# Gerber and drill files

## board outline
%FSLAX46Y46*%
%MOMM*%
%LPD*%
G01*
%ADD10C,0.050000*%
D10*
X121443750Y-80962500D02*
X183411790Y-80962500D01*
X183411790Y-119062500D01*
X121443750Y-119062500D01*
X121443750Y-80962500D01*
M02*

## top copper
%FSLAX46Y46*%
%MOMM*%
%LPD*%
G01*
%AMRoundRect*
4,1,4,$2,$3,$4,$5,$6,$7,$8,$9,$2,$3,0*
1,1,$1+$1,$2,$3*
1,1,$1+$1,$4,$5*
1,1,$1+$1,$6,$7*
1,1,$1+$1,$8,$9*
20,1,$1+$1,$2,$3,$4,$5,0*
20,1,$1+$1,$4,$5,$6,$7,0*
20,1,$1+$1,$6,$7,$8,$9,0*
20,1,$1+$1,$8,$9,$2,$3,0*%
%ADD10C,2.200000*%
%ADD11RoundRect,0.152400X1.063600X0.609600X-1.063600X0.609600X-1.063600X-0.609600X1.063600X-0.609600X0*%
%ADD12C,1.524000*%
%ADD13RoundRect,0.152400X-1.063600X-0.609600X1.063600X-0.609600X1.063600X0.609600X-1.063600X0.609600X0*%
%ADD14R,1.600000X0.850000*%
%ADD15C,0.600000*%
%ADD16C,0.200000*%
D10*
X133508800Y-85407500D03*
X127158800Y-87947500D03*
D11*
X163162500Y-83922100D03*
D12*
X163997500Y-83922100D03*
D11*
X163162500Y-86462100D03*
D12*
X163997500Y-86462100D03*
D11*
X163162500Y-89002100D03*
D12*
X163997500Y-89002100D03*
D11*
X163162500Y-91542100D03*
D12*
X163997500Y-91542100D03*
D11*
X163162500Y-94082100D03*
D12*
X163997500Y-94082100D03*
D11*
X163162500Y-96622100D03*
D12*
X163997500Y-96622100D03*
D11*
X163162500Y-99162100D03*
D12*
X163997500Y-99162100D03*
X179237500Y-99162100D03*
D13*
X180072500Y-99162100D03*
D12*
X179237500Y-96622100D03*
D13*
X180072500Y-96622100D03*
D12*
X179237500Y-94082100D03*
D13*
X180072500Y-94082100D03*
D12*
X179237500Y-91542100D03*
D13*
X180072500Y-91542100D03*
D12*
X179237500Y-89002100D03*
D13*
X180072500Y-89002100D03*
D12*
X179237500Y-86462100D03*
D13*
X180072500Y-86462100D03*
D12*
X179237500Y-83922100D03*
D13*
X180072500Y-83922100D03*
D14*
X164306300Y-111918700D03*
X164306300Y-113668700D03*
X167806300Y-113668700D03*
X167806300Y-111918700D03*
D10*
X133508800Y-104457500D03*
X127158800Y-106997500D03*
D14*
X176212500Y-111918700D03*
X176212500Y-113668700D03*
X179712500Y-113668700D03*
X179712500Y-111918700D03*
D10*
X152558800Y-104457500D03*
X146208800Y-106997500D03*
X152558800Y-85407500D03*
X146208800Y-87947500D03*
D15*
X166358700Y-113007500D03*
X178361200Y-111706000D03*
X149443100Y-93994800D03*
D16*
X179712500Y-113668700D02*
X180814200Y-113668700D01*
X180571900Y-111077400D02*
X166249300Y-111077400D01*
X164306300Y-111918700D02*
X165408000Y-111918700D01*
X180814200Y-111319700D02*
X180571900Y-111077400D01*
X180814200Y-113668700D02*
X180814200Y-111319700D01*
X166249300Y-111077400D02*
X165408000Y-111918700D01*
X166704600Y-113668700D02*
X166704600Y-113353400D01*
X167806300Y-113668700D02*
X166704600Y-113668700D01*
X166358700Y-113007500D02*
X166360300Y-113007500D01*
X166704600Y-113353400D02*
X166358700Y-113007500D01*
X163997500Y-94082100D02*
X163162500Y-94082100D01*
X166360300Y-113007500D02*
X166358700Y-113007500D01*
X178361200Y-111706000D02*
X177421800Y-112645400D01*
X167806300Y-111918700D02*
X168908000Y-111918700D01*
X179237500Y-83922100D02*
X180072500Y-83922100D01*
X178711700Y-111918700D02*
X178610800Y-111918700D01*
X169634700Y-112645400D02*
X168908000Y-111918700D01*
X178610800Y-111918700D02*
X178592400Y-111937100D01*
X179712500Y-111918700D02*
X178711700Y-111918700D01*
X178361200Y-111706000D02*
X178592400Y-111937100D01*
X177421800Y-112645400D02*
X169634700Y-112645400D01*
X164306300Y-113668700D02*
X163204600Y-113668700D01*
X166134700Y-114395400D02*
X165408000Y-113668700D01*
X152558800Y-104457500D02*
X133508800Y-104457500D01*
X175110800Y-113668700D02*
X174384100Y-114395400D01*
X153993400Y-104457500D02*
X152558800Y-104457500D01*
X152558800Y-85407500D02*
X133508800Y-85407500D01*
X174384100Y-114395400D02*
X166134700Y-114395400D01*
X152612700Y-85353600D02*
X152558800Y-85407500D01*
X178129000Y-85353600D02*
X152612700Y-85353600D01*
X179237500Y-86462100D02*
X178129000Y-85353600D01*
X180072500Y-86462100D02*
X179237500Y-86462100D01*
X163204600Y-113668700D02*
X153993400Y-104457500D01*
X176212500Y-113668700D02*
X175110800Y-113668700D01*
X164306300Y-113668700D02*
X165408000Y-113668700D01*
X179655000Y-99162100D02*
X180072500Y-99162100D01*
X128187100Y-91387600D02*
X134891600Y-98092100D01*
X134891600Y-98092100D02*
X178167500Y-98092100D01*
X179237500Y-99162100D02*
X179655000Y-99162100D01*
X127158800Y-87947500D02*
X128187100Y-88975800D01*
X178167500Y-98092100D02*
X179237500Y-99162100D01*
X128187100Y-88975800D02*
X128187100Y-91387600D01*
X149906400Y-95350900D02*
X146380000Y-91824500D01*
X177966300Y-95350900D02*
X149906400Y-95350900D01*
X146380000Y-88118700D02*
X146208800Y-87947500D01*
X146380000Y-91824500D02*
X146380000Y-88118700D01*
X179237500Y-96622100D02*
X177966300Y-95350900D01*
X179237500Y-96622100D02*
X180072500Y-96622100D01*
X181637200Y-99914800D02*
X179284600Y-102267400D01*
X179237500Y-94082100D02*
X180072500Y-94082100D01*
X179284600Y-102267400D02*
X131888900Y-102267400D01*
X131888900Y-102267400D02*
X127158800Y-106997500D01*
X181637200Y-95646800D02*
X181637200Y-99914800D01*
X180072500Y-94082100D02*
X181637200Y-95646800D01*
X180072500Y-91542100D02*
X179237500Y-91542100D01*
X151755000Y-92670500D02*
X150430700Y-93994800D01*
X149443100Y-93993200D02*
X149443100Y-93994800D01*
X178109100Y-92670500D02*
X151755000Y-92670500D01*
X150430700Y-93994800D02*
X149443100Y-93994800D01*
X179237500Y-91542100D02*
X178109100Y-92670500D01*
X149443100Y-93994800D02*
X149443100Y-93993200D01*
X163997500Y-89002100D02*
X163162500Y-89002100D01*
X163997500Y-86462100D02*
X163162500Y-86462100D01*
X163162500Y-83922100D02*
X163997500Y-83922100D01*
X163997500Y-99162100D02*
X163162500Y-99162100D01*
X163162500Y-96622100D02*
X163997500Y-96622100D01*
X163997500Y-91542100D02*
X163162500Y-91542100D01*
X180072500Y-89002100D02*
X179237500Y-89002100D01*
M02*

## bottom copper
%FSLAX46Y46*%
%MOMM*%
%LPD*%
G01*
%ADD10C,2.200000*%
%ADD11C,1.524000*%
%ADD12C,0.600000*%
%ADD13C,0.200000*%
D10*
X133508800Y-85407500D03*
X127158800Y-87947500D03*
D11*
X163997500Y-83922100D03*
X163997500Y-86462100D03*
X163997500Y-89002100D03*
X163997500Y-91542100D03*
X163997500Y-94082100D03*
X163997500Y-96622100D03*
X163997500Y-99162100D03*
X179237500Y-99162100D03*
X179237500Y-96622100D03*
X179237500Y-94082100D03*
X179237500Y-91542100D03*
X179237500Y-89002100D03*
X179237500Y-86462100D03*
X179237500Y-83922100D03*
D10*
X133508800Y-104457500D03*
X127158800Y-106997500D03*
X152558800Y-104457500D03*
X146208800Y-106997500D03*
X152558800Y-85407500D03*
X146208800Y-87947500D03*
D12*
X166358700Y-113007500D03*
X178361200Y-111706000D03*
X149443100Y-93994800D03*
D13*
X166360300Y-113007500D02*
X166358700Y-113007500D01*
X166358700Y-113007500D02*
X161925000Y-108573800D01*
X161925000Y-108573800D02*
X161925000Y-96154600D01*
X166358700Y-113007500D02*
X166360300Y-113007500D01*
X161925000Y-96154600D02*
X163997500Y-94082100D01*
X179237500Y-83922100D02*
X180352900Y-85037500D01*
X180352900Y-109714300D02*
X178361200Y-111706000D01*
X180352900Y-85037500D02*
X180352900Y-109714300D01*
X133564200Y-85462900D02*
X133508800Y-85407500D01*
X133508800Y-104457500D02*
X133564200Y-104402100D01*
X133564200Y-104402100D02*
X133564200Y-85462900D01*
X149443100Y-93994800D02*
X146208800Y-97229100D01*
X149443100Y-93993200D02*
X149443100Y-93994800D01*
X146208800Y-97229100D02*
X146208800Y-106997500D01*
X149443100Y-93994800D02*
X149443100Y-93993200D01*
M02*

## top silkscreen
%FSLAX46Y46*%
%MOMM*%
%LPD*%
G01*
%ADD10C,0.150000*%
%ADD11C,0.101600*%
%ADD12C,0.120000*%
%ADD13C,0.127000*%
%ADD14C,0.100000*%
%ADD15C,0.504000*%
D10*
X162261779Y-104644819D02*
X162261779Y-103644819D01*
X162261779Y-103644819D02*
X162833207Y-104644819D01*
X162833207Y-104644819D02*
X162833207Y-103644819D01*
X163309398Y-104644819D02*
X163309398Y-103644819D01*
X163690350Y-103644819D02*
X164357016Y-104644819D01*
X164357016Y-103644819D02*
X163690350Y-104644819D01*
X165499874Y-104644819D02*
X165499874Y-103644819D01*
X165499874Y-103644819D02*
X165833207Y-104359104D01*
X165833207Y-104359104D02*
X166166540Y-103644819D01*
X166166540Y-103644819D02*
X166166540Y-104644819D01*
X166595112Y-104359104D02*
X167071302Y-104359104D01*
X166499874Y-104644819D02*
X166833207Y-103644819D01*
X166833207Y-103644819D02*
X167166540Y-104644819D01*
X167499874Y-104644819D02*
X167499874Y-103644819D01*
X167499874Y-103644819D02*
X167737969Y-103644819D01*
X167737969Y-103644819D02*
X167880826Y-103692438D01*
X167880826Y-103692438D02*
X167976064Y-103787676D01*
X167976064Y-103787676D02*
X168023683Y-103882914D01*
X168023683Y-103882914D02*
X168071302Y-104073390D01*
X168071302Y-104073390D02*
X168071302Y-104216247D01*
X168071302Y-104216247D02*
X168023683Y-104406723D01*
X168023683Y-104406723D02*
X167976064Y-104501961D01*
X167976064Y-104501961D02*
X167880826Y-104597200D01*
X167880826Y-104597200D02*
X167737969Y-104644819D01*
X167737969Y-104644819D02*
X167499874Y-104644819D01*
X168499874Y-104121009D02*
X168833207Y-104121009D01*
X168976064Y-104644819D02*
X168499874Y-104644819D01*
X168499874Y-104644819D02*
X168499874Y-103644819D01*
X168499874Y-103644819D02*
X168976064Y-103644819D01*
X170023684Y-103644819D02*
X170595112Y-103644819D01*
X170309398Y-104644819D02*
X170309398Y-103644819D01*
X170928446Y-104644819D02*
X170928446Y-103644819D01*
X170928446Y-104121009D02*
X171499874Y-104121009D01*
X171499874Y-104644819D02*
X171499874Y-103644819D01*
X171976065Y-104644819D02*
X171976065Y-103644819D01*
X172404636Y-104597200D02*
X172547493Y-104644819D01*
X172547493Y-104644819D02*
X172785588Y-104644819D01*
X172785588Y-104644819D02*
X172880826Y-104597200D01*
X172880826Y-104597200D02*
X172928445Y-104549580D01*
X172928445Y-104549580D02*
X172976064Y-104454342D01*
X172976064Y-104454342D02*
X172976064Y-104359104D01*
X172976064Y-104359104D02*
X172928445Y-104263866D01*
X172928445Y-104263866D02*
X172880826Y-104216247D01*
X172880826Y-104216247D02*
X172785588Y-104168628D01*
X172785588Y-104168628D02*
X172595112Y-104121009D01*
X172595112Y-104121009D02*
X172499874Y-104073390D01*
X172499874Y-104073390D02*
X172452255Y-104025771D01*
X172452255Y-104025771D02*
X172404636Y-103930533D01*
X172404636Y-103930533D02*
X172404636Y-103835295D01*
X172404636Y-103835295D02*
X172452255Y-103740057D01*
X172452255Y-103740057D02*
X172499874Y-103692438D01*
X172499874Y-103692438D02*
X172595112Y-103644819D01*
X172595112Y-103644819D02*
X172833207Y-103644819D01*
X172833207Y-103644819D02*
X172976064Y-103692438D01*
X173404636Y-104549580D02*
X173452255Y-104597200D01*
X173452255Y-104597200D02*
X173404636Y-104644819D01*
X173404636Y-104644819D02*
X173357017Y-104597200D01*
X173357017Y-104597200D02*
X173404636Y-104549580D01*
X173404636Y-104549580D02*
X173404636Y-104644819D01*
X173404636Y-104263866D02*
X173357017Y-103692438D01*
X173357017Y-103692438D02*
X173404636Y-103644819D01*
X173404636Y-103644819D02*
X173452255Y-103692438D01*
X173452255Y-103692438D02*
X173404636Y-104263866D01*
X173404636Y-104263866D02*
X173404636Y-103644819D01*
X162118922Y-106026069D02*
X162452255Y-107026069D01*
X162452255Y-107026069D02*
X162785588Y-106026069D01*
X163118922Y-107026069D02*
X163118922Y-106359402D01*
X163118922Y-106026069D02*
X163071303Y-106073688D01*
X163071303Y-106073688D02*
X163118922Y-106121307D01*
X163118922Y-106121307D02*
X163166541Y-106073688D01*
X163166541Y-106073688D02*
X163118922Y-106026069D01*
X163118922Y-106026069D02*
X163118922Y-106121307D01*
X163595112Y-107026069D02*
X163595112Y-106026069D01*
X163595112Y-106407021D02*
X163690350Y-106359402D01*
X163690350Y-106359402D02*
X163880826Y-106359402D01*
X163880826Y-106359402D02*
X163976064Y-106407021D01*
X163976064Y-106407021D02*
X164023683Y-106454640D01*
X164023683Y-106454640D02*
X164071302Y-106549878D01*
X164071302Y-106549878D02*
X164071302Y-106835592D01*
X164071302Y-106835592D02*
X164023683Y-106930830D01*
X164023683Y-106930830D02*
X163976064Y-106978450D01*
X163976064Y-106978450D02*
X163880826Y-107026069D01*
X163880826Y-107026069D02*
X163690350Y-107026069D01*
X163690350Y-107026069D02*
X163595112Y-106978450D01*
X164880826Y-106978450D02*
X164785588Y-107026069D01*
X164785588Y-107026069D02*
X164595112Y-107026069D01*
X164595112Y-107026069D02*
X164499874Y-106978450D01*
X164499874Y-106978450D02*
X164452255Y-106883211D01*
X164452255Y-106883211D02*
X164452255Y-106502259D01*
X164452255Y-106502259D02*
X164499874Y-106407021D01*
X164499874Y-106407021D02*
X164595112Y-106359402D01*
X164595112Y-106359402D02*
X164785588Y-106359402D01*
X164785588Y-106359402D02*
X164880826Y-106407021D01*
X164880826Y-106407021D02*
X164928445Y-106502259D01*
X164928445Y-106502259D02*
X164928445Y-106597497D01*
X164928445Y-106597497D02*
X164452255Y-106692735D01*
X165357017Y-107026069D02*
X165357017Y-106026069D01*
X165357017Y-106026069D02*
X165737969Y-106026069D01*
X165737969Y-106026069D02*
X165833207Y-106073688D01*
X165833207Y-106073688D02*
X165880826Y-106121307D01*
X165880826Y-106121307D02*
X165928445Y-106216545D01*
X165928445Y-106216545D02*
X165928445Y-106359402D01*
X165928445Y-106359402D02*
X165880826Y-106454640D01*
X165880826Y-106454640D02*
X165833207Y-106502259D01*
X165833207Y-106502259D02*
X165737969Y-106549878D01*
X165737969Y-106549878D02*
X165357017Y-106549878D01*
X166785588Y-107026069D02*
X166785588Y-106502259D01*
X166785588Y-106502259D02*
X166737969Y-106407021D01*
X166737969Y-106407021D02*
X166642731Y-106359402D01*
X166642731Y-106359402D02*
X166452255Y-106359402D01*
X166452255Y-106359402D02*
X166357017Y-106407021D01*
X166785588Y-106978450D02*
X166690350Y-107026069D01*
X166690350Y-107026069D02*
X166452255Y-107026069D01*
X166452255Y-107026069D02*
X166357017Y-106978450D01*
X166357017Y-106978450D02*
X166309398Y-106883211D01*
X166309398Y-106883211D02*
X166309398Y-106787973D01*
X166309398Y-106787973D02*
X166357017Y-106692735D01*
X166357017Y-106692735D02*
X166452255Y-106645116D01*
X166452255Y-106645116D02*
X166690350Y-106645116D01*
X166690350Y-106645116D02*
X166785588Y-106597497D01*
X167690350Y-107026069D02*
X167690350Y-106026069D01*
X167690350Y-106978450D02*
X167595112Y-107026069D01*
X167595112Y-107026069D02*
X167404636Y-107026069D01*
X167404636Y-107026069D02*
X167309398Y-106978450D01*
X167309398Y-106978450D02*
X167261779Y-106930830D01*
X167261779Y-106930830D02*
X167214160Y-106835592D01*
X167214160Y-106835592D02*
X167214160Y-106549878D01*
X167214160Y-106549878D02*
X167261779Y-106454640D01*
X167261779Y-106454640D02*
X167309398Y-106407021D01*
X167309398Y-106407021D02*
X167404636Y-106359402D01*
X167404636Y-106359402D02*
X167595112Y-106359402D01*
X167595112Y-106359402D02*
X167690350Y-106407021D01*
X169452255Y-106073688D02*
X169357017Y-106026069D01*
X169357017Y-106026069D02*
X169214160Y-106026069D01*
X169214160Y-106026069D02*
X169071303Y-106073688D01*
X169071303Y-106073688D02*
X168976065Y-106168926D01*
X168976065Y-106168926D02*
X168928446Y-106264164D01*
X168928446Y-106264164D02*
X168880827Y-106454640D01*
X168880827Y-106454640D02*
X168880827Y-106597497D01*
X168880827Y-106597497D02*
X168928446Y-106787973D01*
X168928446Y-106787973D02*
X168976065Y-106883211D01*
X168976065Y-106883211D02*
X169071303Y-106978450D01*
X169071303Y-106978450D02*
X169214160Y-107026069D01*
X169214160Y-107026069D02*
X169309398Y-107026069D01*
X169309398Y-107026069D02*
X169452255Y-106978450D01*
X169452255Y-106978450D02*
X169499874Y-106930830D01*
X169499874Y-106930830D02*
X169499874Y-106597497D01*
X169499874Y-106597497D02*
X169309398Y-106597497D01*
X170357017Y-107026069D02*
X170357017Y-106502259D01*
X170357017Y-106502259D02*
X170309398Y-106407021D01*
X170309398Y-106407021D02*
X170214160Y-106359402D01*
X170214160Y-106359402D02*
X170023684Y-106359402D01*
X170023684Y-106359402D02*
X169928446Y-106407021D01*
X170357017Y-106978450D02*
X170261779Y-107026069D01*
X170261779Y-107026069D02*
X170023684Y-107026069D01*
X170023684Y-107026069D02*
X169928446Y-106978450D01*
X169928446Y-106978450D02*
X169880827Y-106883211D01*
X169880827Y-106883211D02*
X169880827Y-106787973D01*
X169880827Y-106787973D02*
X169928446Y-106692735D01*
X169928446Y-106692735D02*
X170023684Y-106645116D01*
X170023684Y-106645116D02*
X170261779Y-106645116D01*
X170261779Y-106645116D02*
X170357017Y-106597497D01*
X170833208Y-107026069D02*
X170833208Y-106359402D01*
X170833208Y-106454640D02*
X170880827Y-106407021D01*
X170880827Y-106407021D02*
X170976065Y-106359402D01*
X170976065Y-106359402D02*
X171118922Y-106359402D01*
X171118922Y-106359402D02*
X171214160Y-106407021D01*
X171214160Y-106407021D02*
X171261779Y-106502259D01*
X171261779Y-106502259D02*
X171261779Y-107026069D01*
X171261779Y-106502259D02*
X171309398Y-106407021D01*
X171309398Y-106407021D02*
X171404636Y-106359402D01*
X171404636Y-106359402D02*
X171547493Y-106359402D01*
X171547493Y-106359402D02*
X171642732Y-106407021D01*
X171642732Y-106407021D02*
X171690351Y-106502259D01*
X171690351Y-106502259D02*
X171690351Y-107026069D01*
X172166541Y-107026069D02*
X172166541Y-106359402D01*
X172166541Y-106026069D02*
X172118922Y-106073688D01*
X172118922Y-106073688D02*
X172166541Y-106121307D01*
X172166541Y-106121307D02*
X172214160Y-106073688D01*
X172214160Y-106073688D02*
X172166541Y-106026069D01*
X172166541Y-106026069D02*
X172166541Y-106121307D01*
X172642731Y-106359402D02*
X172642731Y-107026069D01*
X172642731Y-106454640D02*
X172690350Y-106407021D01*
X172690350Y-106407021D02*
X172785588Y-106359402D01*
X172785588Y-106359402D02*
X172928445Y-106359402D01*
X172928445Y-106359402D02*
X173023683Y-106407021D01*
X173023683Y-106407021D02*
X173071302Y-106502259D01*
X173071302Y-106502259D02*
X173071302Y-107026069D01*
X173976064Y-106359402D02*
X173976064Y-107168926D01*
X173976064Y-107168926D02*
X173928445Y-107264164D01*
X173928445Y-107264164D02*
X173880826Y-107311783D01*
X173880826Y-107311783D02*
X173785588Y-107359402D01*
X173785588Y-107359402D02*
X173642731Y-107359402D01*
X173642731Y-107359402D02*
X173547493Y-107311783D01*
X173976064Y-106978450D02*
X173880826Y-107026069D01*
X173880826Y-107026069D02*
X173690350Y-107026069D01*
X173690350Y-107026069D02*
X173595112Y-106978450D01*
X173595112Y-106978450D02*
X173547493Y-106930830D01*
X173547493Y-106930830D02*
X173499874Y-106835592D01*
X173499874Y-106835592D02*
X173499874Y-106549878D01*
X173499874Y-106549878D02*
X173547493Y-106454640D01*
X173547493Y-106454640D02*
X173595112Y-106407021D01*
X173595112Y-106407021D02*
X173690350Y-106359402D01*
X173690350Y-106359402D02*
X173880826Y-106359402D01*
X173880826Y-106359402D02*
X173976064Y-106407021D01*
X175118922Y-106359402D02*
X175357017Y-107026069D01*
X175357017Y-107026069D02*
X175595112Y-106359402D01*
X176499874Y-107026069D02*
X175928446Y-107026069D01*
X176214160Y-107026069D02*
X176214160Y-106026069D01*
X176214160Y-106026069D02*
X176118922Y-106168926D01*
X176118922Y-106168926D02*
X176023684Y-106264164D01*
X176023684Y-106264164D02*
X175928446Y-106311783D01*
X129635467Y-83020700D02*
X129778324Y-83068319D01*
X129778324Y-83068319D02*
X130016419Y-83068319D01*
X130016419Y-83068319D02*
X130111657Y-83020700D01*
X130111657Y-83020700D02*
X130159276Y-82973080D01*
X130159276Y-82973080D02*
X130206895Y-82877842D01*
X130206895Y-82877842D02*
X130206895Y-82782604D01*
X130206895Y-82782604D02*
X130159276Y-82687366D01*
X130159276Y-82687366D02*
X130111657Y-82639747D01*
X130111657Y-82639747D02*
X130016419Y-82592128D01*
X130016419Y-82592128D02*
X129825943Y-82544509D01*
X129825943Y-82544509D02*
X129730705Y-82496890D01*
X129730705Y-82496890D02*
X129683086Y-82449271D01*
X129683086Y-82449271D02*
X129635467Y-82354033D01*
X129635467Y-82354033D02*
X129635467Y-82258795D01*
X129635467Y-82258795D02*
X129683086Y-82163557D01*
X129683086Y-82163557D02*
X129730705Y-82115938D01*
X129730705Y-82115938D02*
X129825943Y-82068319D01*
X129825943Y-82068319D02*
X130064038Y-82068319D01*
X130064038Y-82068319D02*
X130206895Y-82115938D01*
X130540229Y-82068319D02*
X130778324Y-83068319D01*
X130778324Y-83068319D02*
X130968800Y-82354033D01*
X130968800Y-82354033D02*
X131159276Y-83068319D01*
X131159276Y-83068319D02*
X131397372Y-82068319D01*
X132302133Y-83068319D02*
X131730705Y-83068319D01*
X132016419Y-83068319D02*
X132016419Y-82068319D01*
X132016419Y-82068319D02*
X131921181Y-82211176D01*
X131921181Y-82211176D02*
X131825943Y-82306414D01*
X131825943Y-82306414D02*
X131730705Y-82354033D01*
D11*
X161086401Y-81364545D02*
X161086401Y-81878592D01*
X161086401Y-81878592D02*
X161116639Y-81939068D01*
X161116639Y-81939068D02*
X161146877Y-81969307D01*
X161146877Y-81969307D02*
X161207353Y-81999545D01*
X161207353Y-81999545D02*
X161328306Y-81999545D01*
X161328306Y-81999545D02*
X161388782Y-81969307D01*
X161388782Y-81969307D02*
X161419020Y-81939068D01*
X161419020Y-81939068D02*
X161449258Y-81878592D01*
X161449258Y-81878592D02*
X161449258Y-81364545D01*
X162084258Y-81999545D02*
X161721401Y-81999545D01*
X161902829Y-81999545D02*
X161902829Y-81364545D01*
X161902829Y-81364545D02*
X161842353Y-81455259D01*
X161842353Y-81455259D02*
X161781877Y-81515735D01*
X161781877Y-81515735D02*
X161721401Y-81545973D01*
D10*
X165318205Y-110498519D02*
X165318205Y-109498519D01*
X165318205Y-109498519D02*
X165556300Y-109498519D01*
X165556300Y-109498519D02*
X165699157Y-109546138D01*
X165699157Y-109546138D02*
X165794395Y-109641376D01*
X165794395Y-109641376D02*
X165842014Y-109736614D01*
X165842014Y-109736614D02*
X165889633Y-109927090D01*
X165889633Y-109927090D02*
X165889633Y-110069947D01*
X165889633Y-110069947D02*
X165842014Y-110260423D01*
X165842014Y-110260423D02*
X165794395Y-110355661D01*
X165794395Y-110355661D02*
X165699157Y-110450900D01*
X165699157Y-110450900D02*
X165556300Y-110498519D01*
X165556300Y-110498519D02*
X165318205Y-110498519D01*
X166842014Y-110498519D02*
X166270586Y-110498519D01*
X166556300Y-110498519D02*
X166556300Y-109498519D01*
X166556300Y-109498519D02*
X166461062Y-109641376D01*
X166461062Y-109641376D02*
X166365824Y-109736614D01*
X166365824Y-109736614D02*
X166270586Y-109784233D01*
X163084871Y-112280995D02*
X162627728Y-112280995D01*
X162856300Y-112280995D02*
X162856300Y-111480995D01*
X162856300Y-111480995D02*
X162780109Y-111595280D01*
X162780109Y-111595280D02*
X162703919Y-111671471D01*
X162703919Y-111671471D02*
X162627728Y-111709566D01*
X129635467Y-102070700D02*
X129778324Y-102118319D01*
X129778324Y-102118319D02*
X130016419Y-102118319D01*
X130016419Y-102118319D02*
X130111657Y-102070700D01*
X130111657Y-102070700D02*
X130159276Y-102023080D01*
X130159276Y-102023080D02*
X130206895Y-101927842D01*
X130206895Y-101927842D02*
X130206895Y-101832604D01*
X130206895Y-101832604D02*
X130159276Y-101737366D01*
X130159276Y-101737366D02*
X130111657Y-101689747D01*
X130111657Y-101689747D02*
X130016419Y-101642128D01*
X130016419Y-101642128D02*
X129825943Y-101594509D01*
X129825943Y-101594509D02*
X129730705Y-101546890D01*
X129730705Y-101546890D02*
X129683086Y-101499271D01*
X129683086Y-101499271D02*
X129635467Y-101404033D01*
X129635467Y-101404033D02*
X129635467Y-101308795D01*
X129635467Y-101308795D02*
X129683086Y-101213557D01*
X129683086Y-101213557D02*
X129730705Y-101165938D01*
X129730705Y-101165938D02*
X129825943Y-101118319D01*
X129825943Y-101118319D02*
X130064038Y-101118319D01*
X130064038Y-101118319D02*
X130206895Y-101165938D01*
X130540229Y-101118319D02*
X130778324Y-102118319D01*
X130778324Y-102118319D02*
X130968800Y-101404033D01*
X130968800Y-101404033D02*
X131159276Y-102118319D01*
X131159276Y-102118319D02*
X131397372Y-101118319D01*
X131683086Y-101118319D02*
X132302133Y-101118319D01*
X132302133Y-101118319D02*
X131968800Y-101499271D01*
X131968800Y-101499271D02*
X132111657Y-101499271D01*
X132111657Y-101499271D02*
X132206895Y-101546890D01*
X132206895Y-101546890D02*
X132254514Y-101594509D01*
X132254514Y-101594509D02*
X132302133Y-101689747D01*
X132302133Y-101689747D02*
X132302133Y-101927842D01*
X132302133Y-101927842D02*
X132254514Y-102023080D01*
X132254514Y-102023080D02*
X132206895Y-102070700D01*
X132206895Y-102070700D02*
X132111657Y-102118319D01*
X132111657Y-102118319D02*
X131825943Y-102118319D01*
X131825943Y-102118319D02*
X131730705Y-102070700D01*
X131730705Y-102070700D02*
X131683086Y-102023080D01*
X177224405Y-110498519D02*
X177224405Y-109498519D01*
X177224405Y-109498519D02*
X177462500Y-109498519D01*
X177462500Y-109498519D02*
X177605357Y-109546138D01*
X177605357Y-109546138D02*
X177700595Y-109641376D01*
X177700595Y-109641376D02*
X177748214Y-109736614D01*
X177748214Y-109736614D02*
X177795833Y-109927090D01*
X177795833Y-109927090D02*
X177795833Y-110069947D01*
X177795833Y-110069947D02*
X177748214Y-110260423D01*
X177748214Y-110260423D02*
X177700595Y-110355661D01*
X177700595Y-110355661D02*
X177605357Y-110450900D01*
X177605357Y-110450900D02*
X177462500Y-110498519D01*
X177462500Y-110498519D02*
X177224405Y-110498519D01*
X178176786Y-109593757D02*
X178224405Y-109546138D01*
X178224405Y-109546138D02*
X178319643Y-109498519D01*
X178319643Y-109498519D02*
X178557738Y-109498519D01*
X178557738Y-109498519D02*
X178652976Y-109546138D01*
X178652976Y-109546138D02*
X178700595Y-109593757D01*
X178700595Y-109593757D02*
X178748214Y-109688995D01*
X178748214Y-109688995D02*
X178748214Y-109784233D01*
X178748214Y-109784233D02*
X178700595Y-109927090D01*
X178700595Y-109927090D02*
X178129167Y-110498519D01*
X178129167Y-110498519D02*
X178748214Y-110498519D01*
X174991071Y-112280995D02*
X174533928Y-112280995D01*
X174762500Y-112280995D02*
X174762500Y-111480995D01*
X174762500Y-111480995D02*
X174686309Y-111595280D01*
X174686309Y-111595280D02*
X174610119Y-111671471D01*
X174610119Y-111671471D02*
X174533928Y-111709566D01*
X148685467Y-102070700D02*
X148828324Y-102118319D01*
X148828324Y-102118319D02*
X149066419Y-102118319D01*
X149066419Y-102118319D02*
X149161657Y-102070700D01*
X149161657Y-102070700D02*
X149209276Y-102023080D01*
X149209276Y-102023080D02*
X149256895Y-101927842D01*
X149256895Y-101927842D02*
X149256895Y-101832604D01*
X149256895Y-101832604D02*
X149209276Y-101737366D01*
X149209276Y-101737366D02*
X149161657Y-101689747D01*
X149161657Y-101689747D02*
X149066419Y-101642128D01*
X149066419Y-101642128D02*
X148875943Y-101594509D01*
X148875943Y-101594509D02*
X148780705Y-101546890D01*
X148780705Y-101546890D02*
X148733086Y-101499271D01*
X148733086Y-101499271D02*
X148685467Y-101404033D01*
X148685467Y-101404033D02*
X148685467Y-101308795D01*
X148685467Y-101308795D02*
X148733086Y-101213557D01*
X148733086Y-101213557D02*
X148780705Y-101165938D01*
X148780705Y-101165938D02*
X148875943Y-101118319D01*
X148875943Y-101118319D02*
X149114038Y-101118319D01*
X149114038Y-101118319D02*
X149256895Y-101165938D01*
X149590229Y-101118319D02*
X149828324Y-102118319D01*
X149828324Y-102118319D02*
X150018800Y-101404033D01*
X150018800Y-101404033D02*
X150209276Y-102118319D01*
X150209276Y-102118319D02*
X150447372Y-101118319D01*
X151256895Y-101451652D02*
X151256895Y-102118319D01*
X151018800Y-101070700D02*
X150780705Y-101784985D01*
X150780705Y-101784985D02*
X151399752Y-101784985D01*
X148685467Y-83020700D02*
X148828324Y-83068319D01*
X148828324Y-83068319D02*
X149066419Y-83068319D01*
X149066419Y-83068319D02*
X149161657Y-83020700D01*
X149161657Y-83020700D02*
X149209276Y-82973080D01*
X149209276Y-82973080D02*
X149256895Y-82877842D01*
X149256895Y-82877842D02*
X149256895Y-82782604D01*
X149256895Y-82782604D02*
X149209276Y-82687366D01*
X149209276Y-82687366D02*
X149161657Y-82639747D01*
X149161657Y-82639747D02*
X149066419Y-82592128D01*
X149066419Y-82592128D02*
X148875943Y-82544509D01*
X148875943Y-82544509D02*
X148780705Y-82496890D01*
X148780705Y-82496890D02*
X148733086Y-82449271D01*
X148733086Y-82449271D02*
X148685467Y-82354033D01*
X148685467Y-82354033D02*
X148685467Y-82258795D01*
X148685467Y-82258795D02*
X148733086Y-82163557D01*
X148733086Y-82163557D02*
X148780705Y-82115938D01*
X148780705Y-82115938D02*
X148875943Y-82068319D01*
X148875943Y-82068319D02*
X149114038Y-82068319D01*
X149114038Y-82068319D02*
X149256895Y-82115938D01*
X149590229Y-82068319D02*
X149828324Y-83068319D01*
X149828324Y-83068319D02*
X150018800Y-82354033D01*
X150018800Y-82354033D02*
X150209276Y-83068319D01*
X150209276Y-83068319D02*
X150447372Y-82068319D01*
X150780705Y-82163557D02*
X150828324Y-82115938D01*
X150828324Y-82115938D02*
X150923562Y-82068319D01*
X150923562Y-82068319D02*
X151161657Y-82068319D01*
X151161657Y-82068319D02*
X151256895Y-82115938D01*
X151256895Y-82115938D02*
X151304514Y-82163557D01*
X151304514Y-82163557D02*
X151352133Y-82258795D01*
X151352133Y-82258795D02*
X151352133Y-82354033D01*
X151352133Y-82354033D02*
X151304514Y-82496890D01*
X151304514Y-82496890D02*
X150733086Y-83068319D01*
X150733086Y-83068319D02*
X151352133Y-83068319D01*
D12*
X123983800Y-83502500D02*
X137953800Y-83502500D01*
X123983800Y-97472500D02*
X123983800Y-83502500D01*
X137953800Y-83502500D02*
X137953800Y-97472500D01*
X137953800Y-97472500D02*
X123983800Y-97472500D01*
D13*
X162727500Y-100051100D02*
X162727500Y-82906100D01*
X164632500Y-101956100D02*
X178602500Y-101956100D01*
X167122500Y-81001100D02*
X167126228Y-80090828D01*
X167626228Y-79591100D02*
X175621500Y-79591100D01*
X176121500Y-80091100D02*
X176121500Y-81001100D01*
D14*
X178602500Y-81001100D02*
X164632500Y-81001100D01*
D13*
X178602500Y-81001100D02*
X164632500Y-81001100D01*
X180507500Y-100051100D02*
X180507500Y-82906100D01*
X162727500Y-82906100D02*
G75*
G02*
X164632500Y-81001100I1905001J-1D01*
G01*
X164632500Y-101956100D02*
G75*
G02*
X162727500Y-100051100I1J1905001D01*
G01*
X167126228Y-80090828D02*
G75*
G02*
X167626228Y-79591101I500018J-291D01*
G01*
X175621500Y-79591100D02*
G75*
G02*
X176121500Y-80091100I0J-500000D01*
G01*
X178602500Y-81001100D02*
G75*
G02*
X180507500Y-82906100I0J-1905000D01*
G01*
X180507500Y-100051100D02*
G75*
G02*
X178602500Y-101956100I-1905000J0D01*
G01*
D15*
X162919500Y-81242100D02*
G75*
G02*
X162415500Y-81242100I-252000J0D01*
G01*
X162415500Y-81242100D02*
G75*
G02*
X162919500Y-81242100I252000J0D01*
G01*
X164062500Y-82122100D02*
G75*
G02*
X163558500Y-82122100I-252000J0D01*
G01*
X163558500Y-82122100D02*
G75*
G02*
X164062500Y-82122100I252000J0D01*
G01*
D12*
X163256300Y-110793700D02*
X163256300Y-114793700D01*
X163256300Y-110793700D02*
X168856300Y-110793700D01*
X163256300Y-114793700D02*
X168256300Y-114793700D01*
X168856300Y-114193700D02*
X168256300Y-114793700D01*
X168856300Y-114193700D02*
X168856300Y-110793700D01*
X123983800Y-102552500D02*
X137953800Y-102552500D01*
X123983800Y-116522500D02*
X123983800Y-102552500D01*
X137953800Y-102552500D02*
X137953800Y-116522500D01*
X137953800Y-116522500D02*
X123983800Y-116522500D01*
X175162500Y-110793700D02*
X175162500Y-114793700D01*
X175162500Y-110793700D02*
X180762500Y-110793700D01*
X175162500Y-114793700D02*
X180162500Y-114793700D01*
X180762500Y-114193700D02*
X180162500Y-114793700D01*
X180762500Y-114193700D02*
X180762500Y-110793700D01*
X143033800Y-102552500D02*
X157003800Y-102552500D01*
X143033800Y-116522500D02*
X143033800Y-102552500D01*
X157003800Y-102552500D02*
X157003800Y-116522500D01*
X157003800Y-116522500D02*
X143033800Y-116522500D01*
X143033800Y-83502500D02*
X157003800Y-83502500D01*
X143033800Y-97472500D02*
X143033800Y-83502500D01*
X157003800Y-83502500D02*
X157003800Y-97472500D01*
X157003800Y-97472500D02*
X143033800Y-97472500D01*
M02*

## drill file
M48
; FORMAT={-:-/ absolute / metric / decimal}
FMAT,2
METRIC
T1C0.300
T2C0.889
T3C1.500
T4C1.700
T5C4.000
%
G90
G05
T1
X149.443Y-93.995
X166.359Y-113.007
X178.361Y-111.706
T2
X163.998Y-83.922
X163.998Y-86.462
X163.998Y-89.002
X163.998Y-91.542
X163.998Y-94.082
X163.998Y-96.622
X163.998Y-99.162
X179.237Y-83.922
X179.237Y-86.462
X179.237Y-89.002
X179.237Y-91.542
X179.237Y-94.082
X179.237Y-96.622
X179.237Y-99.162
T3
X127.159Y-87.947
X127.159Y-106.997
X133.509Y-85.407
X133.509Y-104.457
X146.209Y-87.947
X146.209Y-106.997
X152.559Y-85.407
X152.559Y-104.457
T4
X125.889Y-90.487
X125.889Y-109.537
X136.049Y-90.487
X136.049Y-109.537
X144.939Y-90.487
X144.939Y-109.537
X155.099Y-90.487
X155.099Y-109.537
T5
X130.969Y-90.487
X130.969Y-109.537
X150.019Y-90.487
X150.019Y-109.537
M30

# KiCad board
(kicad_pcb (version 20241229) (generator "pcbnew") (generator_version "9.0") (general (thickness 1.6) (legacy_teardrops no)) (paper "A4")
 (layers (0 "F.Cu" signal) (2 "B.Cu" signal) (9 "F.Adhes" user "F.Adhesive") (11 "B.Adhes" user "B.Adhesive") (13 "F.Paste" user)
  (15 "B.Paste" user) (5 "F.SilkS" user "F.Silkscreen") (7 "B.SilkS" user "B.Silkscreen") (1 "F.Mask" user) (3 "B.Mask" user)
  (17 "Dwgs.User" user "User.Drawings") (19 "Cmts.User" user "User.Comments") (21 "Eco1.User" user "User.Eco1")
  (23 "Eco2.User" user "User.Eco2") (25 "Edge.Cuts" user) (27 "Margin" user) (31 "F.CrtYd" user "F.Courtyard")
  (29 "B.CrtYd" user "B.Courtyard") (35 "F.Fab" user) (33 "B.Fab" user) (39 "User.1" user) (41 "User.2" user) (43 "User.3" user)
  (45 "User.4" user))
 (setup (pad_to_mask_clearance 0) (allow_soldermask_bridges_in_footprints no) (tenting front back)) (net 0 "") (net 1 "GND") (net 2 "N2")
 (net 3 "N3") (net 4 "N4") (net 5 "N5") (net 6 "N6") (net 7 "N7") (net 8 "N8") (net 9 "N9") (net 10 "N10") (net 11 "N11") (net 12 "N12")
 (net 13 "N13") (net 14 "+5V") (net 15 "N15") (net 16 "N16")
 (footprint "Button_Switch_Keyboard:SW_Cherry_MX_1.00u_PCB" (layer "F.Cu") (at 133.5088 85.4075)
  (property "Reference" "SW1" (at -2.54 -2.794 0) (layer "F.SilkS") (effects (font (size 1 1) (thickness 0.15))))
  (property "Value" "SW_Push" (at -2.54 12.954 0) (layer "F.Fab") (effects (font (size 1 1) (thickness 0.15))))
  (fp_line (start -9.525 -1.905) (end 4.445 -1.905) (stroke (width 0.12) (type solid)) (layer "F.SilkS"))
  (fp_line (start -9.525 12.065) (end -9.525 -1.905) (stroke (width 0.12) (type solid)) (layer "F.SilkS"))
  (fp_line (start 4.445 -1.905) (end 4.445 12.065) (stroke (width 0.12) (type solid)) (layer "F.SilkS"))
  (fp_line (start 4.445 12.065) (end -9.525 12.065) (stroke (width 0.12) (type solid)) (layer "F.SilkS"))
  (pad "" np_thru_hole circle (at -7.62 5.08) (size 1.7 1.7) (drill 1.7) (layers "*.Cu" "*.Mask"))
  (pad "" np_thru_hole circle (at -2.54 5.08) (size 4 4) (drill 4) (layers "*.Cu" "*.Mask"))
  (pad "" np_thru_hole circle (at 2.54 5.08) (size 1.7 1.7) (drill 1.7) (layers "*.Cu" "*.Mask"))
  (pad "1" thru_hole circle (at 0 0) (size 2.2 2.2) (drill 1.5) (layers "*.Cu" "*.Mask") (remove_unused_layers no) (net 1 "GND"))
  (pad "2" thru_hole circle (at -6.35 2.54) (size 2.2 2.2) (drill 1.5) (layers "*.Cu" "*.Mask") (remove_unused_layers no) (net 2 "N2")))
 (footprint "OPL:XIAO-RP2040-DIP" (layer "F.Cu") (at 171.6175 91.5421)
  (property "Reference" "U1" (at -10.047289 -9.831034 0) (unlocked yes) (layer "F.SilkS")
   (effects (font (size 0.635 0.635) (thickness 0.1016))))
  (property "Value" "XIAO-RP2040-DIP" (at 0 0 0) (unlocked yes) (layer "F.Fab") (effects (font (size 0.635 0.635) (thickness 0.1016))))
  (fp_line (start -8.89 8.509) (end -8.89 -8.636) (stroke (width 0.127) (type solid)) (layer "F.SilkS"))
  (fp_line (start -6.985 10.414) (end 6.985 10.414) (stroke (width 0.127) (type solid)) (layer "F.SilkS"))
  (fp_line (start -4.495 -10.541) (end -4.491272 -11.451272) (stroke (width 0.127) (type solid)) (layer "F.SilkS"))
  (fp_line (start -3.991272 -11.951) (end 4.004 -11.951) (stroke (width 0.127) (type solid)) (layer "F.SilkS"))
  (fp_line (start 4.504 -11.451) (end 4.504 -10.541) (stroke (width 0.127) (type solid)) (layer "F.SilkS"))
  (fp_line (start 6.985 -10.541) (end -6.985 -10.541) (stroke (width 0.1) (type solid)) (layer "F.SilkS"))
  (fp_line (start 6.985 -10.541) (end -6.985 -10.541) (stroke (width 0.127) (type solid)) (layer "F.SilkS"))
  (fp_line (start 8.89 8.509) (end 8.89 -8.636) (stroke (width 0.127) (type solid)) (layer "F.SilkS"))
  (fp_arc (start -8.89 -8.636) (mid -8.332038 -9.983038) (end -6.985 -10.541) (stroke (width 0.127) (type solid)) (layer "F.SilkS"))
  (fp_arc (start -6.985 10.414) (mid -8.332038 9.856038) (end -8.89 8.509) (stroke (width 0.127) (type solid)) (layer "F.SilkS"))
  (fp_arc (start -4.491272 -11.451272) (mid -4.344728 -11.80464) (end -3.991272 -11.951) (stroke (width 0.127) (type default))
   (layer "F.SilkS"))
  (fp_arc (start 4.004 -11.951) (mid 4.357553 -11.804553) (end 4.504 -11.451) (stroke (width 0.127) (type default)) (layer "F.SilkS"))
  (fp_arc (start 6.985 -10.541) (mid 8.332038 -9.983038) (end 8.89 -8.636) (stroke (width 0.127) (type solid)) (layer "F.SilkS"))
  (fp_arc (start 8.89 8.509) (mid 8.332038 9.856038) (end 6.985 10.414) (stroke (width 0.127) (type solid)) (layer "F.SilkS"))
  (fp_circle (center -8.95 -10.3) (end -8.95 -10.554) (stroke (width 0.5) (type solid)) (fill yes) (layer "F.SilkS"))
  (fp_circle (center -7.807 -9.42) (end -7.807 -9.674) (stroke (width 0.5) (type solid)) (fill yes) (layer "F.SilkS"))
  (pad "1" smd roundrect (at -8.455 -7.62 180) (size 2.432 1.524) (layers "F.Cu" "F.Mask") (roundrect_rratio 0.1) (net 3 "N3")
   (thermal_bridge_angle 45))
  (pad "1" thru_hole circle (at -7.62 -7.62 180) (size 1.524 1.524) (drill 0.889) (layers "*.Cu" "*.Mask") (remove_unused_layers no)
   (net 3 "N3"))
  (pad "2" smd roundrect (at -8.455 -5.08 180) (size 2.432 1.524) (layers "F.Cu" "F.Mask") (roundrect_rratio 0.1) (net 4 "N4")
   (thermal_bridge_angle 45))
  (pad "2" thru_hole circle (at -7.62 -5.08 180) (size 1.524 1.524) (drill 0.889) (layers "*.Cu" "*.Mask") (remove_unused_layers no)
   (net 4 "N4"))
  (pad "3" smd roundrect (at -8.455 -2.54 180) (size 2.432 1.524) (layers "F.Cu" "F.Mask") (roundrect_rratio 0.1) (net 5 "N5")
   (thermal_bridge_angle 45))
  (pad "3" thru_hole circle (at -7.62 -2.54 180) (size 1.524 1.524) (drill 0.889) (layers "*.Cu" "*.Mask") (remove_unused_layers no)
   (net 5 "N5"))
  (pad "4" smd roundrect (at -8.455 0 180) (size 2.432 1.524) (layers "F.Cu" "F.Mask") (roundrect_rratio 0.1) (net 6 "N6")
   (thermal_bridge_angle 45))
  (pad "4" thru_hole circle (at -7.62 0 180) (size 1.524 1.524) (drill 0.889) (layers "*.Cu" "*.Mask") (remove_unused_layers no)
   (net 6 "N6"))
  (pad "5" smd roundrect (at -8.455 2.54 180) (size 2.432 1.524) (layers "F.Cu" "F.Mask") (roundrect_rratio 0.1) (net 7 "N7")
   (thermal_bridge_angle 45))
  (pad "5" thru_hole circle (at -7.62 2.54 180) (size 1.524 1.524) (drill 0.889) (layers "*.Cu" "*.Mask") (remove_unused_layers no)
   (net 7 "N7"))
  (pad "6" smd roundrect (at -8.455 5.08 180) (size 2.432 1.524) (layers "F.Cu" "F.Mask") (roundrect_rratio 0.1) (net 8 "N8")
   (thermal_bridge_angle 45))
  (pad "6" thru_hole circle (at -7.62 5.08 180) (size 1.524 1.524) (drill 0.889) (layers "*.Cu" "*.Mask") (remove_unused_layers no)
   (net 8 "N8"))
  (pad "7" smd roundrect (at -8.455 7.62 180) (size 2.432 1.524) (layers "F.Cu" "F.Mask") (roundrect_rratio 0.1) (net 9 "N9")
   (thermal_bridge_angle 45))
  (pad "7" thru_hole circle (at -7.62 7.62 180) (size 1.524 1.524) (drill 0.889) (layers "*.Cu" "*.Mask") (remove_unused_layers no)
   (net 9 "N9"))
  (pad "8" thru_hole circle (at 7.62 7.62) (size 1.524 1.524) (drill 0.889) (layers "*.Cu" "*.Mask") (remove_unused_layers no) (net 2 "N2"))
  (pad "8" smd roundrect (at 8.455 7.62) (size 2.432 1.524) (layers "F.Cu" "F.Mask") (roundrect_rratio 0.1) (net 2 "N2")
   (thermal_bridge_angle 45))
  (pad "9" thru_hole circle (at 7.62 5.08) (size 1.524 1.524) (drill 0.889) (layers "*.Cu" "*.Mask") (remove_unused_layers no)
   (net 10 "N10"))
  (pad "9" smd roundrect (at 8.455 5.08) (size 2.432 1.524) (layers "F.Cu" "F.Mask") (roundrect_rratio 0.1) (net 10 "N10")
   (thermal_bridge_angle 45))
  (pad "10" thru_hole circle (at 7.62 2.54) (size 1.524 1.524) (drill 0.889) (layers "*.Cu" "*.Mask") (remove_unused_layers no)
   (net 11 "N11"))
  (pad "10" smd roundrect (at 8.455 2.54) (size 2.432 1.524) (layers "F.Cu" "F.Mask") (roundrect_rratio 0.1) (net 11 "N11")
   (thermal_bridge_angle 45))
  (pad "11" thru_hole circle (at 7.62 0) (size 1.524 1.524) (drill 0.889) (layers "*.Cu" "*.Mask") (remove_unused_layers no) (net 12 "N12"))
  (pad "11" smd roundrect (at 8.455 0) (size 2.432 1.524) (layers "F.Cu" "F.Mask") (roundrect_rratio 0.1) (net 12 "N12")
   (thermal_bridge_angle 45))
  (pad "12" thru_hole circle (at 7.62 -2.54) (size 1.524 1.524) (drill 0.889) (layers "*.Cu" "*.Mask") (remove_unused_layers no)
   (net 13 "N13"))
  (pad "12" smd roundrect (at 8.455 -2.54) (size 2.432 1.524) (layers "F.Cu" "F.Mask") (roundrect_rratio 0.1) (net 13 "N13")
   (thermal_bridge_angle 45))
  (pad "13" thru_hole circle (at 7.62 -5.08) (size 1.524 1.524) (drill 0.889) (layers "*.Cu" "*.Mask") (remove_unused_layers no)
   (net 1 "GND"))
  (pad "13" smd roundrect (at 8.455 -5.08) (size 2.432 1.524) (layers "F.Cu" "F.Mask") (roundrect_rratio 0.1) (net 1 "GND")
   (thermal_bridge_angle 45))
  (pad "14" thru_hole circle (at 7.62 -7.62) (size 1.524 1.524) (drill 0.889) (layers "*.Cu" "*.Mask") (remove_unused_layers no)
   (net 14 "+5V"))
  (pad "14" smd roundrect (at 8.455 -7.62) (size 2.432 1.524) (layers "F.Cu" "F.Mask") (roundrect_rratio 0.1) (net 14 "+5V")
   (thermal_bridge_angle 45)))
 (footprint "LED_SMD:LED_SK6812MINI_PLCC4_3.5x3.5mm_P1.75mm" (layer "F.Cu") (at 166.0563 112.7937)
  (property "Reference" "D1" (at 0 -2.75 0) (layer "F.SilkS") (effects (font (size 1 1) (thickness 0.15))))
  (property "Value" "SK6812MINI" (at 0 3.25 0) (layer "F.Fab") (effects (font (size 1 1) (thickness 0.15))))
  (fp_line (start -2.8 -2) (end -2.8 2) (stroke (width 0.12) (type default)) (layer "F.SilkS"))
  (fp_line (start -2.8 -2) (end 2.8 -2) (stroke (width 0.12) (type solid)) (layer "F.SilkS"))
  (fp_line (start -2.8 2) (end 2.2 2) (stroke (width 0.12) (type solid)) (layer "F.SilkS"))
  (fp_line (start 2.8 1.4) (end 2.2 2) (stroke (width 0.12) (type default)) (layer "F.SilkS"))
  (fp_line (start 2.8 1.4) (end 2.8 -2) (stroke (width 0.12) (type solid)) (layer "F.SilkS"))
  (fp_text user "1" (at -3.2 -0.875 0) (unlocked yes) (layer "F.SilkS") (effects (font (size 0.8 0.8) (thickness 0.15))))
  (pad "1" smd rect (at -1.75 -0.875) (size 1.6 0.85) (layers "F.Cu" "F.Mask" "F.Paste") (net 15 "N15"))
  (pad "2" smd rect (at -1.75 0.875) (size 1.6 0.85) (layers "F.Cu" "F.Mask" "F.Paste") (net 1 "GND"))
  (pad "3" smd rect (at 1.75 0.875) (size 1.6 0.85) (layers "F.Cu" "F.Mask" "F.Paste") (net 7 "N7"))
  (pad "4" smd rect (at 1.75 -0.875) (size 1.6 0.85) (layers "F.Cu" "F.Mask" "F.Paste") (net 14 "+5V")))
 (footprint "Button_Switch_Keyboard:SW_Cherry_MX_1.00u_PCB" (layer "F.Cu") (at 133.5088 104.4575)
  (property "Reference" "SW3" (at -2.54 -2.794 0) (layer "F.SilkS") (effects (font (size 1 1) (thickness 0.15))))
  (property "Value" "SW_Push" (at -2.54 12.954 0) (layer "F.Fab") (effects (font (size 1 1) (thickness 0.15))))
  (fp_line (start -9.525 -1.905) (end 4.445 -1.905) (stroke (width 0.12) (type solid)) (layer "F.SilkS"))
  (fp_line (start -9.525 12.065) (end -9.525 -1.905) (stroke (width 0.12) (type solid)) (layer "F.SilkS"))
  (fp_line (start 4.445 -1.905) (end 4.445 12.065) (stroke (width 0.12) (type solid)) (layer "F.SilkS"))
  (fp_line (start 4.445 12.065) (end -9.525 12.065) (stroke (width 0.12) (type solid)) (layer "F.SilkS"))
  (pad "" np_thru_hole circle (at -7.62 5.08) (size 1.7 1.7) (drill 1.7) (layers "*.Cu" "*.Mask"))
  (pad "" np_thru_hole circle (at -2.54 5.08) (size 4 4) (drill 4) (layers "*.Cu" "*.Mask"))
  (pad "" np_thru_hole circle (at 2.54 5.08) (size 1.7 1.7) (drill 1.7) (layers "*.Cu" "*.Mask"))
  (pad "1" thru_hole circle (at 0 0) (size 2.2 2.2) (drill 1.5) (layers "*.Cu" "*.Mask") (remove_unused_layers no) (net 1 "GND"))
  (pad "2" thru_hole circle (at -6.35 2.54) (size 2.2 2.2) (drill 1.5) (layers "*.Cu" "*.Mask") (remove_unused_layers no) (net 11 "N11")))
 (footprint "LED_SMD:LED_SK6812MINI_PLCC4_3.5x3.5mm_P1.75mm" (layer "F.Cu") (at 177.9625 112.7937)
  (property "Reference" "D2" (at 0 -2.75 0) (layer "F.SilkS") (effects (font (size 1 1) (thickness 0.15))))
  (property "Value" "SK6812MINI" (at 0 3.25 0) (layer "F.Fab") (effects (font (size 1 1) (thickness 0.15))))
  (fp_line (start -2.8 -2) (end -2.8 2) (stroke (width 0.12) (type default)) (layer "F.SilkS"))
  (fp_line (start -2.8 -2) (end 2.8 -2) (stroke (width 0.12) (type solid)) (layer "F.SilkS"))
  (fp_line (start -2.8 2) (end 2.2 2) (stroke (width 0.12) (type solid)) (layer "F.SilkS"))
  (fp_line (start 2.8 1.4) (end 2.2 2) (stroke (width 0.12) (type default)) (layer "F.SilkS"))
  (fp_line (start 2.8 1.4) (end 2.8 -2) (stroke (width 0.12) (type solid)) (layer "F.SilkS"))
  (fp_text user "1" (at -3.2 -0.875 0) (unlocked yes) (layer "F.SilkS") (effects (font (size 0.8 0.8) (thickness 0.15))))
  (pad "1" smd rect (at -1.75 -0.875) (size 1.6 0.85) (layers "F.Cu" "F.Mask" "F.Paste") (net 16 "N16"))
  (pad "2" smd rect (at -1.75 0.875) (size 1.6 0.85) (layers "F.Cu" "F.Mask" "F.Paste") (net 1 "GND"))
  (pad "3" smd rect (at 1.75 0.875) (size 1.6 0.85) (layers "F.Cu" "F.Mask" "F.Paste") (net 15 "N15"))
  (pad "4" smd rect (at 1.75 -0.875) (size 1.6 0.85) (layers "F.Cu" "F.Mask" "F.Paste") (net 14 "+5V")))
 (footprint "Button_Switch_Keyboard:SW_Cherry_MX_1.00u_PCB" (layer "F.Cu") (at 152.5588 104.4575)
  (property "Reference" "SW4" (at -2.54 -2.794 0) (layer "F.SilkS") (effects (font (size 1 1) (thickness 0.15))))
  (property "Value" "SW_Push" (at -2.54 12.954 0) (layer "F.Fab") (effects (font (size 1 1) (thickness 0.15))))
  (fp_line (start -9.525 -1.905) (end 4.445 -1.905) (stroke (width 0.12) (type solid)) (layer "F.SilkS"))
  (fp_line (start -9.525 12.065) (end -9.525 -1.905) (stroke (width 0.12) (type solid)) (layer "F.SilkS"))
  (fp_line (start 4.445 -1.905) (end 4.445 12.065) (stroke (width 0.12) (type solid)) (layer "F.SilkS"))
  (fp_line (start 4.445 12.065) (end -9.525 12.065) (stroke (width 0.12) (type solid)) (layer "F.SilkS"))
  (pad "" np_thru_hole circle (at -7.62 5.08) (size 1.7 1.7) (drill 1.7) (layers "*.Cu" "*.Mask"))
  (pad "" np_thru_hole circle (at -2.54 5.08) (size 4 4) (drill 4) (layers "*.Cu" "*.Mask"))
  (pad "" np_thru_hole circle (at 2.54 5.08) (size 1.7 1.7) (drill 1.7) (layers "*.Cu" "*.Mask"))
  (pad "1" thru_hole circle (at 0 0) (size 2.2 2.2) (drill 1.5) (layers "*.Cu" "*.Mask") (remove_unused_layers no) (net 1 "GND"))
  (pad "2" thru_hole circle (at -6.35 2.54) (size 2.2 2.2) (drill 1.5) (layers "*.Cu" "*.Mask") (remove_unused_layers no) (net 12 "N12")))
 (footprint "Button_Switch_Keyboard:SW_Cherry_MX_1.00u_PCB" (layer "F.Cu") (at 152.5588 85.4075)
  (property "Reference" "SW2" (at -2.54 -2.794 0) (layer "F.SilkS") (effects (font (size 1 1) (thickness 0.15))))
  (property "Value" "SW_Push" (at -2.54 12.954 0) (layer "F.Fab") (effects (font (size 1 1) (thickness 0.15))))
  (fp_line (start -9.525 -1.905) (end 4.445 -1.905) (stroke (width 0.12) (type solid)) (layer "F.SilkS"))
  (fp_line (start -9.525 12.065) (end -9.525 -1.905) (stroke (width 0.12) (type solid)) (layer "F.SilkS"))
  (fp_line (start 4.445 -1.905) (end 4.445 12.065) (stroke (width 0.12) (type solid)) (layer "F.SilkS"))
  (fp_line (start 4.445 12.065) (end -9.525 12.065) (stroke (width 0.12) (type solid)) (layer "F.SilkS"))
  (pad "" np_thru_hole circle (at -7.62 5.08) (size 1.7 1.7) (drill 1.7) (layers "*.Cu" "*.Mask"))
  (pad "" np_thru_hole circle (at -2.54 5.08) (size 4 4) (drill 4) (layers "*.Cu" "*.Mask"))
  (pad "" np_thru_hole circle (at 2.54 5.08) (size 1.7 1.7) (drill 1.7) (layers "*.Cu" "*.Mask"))
  (pad "1" thru_hole circle (at 0 0) (size 2.2 2.2) (drill 1.5) (layers "*.Cu" "*.Mask") (remove_unused_layers no) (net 1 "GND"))
  (pad "2" thru_hole circle (at -6.35 2.54) (size 2.2 2.2) (drill 1.5) (layers "*.Cu" "*.Mask") (remove_unused_layers no) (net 10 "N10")))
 (gr_rect (start 121.44375 80.9625) (end 183.41179 119.0625) (stroke (width 0.05) (type default)) (fill no) (layer "Edge.Cuts"))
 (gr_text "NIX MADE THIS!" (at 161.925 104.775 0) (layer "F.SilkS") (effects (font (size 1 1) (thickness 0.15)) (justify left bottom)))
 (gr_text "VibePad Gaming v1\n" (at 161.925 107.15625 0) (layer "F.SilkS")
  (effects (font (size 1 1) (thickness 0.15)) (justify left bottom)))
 (segment (start 179.7125 113.6687) (end 180.8142 113.6687) (width 0.2) (layer "F.Cu") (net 15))
 (segment (start 180.5719 111.0774) (end 166.2493 111.0774) (width 0.2) (layer "F.Cu") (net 15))
 (segment (start 164.3063 111.9187) (end 165.408 111.9187) (width 0.2) (layer "F.Cu") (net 15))
 (segment (start 180.8142 111.3197) (end 180.5719 111.0774) (width 0.2) (layer "F.Cu") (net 15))
 (segment (start 180.8142 113.6687) (end 180.8142 111.3197) (width 0.2) (layer "F.Cu") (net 15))
 (segment (start 166.2493 111.0774) (end 165.408 111.9187) (width 0.2) (layer "F.Cu") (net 15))
 (segment (start 166.7046 113.6687) (end 166.7046 113.3534) (width 0.2) (layer "F.Cu") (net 7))
 (segment (start 167.8063 113.6687) (end 166.7046 113.6687) (width 0.2) (layer "F.Cu") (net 7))
 (segment (start 166.3587 113.0075) (end 166.3603 113.0075) (width 0.2) (layer "F.Cu") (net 7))
 (segment (start 166.7046 113.3534) (end 166.3587 113.0075) (width 0.2) (layer "F.Cu") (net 7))
 (segment (start 163.9975 94.0821) (end 163.1625 94.0821) (width 0.2) (layer "F.Cu") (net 7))
 (segment (start 166.3603 113.0075) (end 166.3587 113.0075) (width 0.2) (layer "F.Cu") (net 7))
 (via (at 166.3587 113.0075) (size 0.6) (drill 0.3) (layers "F.Cu" "B.Cu") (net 7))
 (segment (start 166.3603 113.0075) (end 166.3587 113.0075) (width 0.2) (layer "B.Cu") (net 7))
 (segment (start 166.3587 113.0075) (end 161.925 108.5738) (width 0.2) (layer "B.Cu") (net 7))
 (segment (start 161.925 108.5738) (end 161.925 96.1546) (width 0.2) (layer "B.Cu") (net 7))
 (segment (start 166.3587 113.0075) (end 166.3603 113.0075) (width 0.2) (layer "B.Cu") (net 7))
 (segment (start 161.925 96.1546) (end 163.9975 94.0821) (width 0.2) (layer "B.Cu") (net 7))
 (segment (start 178.3612 111.706) (end 177.4218 112.6454) (width 0.2) (layer "F.Cu") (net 14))
 (segment (start 167.8063 111.9187) (end 168.908 111.9187) (width 0.2) (layer "F.Cu") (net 14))
 (segment (start 179.2375 83.9221) (end 180.0725 83.9221) (width 0.2) (layer "F.Cu") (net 14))
 (segment (start 178.7117 111.9187) (end 178.6108 111.9187) (width 0.2) (layer "F.Cu") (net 14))
 (segment (start 169.6347 112.6454) (end 168.908 111.9187) (width 0.2) (layer "F.Cu") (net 14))
 (segment (start 178.6108 111.9187) (end 178.5924 111.9371) (width 0.2) (layer "F.Cu") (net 14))
 (segment (start 179.7125 111.9187) (end 178.7117 111.9187) (width 0.2) (layer "F.Cu") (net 14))
 (segment (start 178.3612 111.706) (end 178.5924 111.9371) (width 0.2) (layer "F.Cu") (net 14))
 (segment (start 177.4218 112.6454) (end 169.6347 112.6454) (width 0.2) (layer "F.Cu") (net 14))
 (via (at 178.3612 111.706) (size 0.6) (drill 0.3) (layers "F.Cu" "B.Cu") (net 14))
 (segment (start 179.2375 83.9221) (end 180.3529 85.0375) (width 0.2) (layer "B.Cu") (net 14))
 (segment (start 180.3529 109.7143) (end 178.3612 111.706) (width 0.2) (layer "B.Cu") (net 14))
 (segment (start 180.3529 85.0375) (end 180.3529 109.7143) (width 0.2) (layer "B.Cu") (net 14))
 (segment (start 164.3063 113.6687) (end 163.2046 113.6687) (width 0.2) (layer "F.Cu") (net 1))
 (segment (start 166.1347 114.3954) (end 165.408 113.6687) (width 0.2) (layer "F.Cu") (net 1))
 (segment (start 152.5588 104.4575) (end 133.5088 104.4575) (width 0.2) (layer "F.Cu") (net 1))
 (segment (start 175.1108 113.6687) (end 174.3841 114.3954) (width 0.2) (layer "F.Cu") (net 1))
 (segment (start 153.9934 104.4575) (end 152.5588 104.4575) (width 0.2) (layer "F.Cu") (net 1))
 (segment (start 152.5588 85.4075) (end 133.5088 85.4075) (width 0.2) (layer "F.Cu") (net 1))
 (segment (start 174.3841 114.3954) (end 166.1347 114.3954) (width 0.2) (layer "F.Cu") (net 1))
 (segment (start 152.6127 85.3536) (end 152.5588 85.4075) (width 0.2) (layer "F.Cu") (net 1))
 (segment (start 178.129 85.3536) (end 152.6127 85.3536) (width 0.2) (layer "F.Cu") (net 1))
 (segment (start 179.2375 86.4621) (end 178.129 85.3536) (width 0.2) (layer "F.Cu") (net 1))
 (segment (start 180.0725 86.4621) (end 179.2375 86.4621) (width 0.2) (layer "F.Cu") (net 1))
 (segment (start 163.2046 113.6687) (end 153.9934 104.4575) (width 0.2) (layer "F.Cu") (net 1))
 (segment (start 176.2125 113.6687) (end 175.1108 113.6687) (width 0.2) (layer "F.Cu") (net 1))
 (segment (start 164.3063 113.6687) (end 165.408 113.6687) (width 0.2) (layer "F.Cu") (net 1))
 (segment (start 133.5642 85.4629) (end 133.5088 85.4075) (width 0.2) (layer "B.Cu") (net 1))
 (segment (start 133.5088 104.4575) (end 133.5642 104.4021) (width 0.2) (layer "B.Cu") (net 1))
 (segment (start 133.5642 104.4021) (end 133.5642 85.4629) (width 0.2) (layer "B.Cu") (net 1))
 (segment (start 179.655 99.1621) (end 180.0725 99.1621) (width 0.2) (layer "F.Cu") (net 2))
 (segment (start 128.1871 91.3876) (end 134.8916 98.0921) (width 0.2) (layer "F.Cu") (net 2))
 (segment (start 134.8916 98.0921) (end 178.1675 98.0921) (width 0.2) (layer "F.Cu") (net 2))
 (segment (start 179.2375 99.1621) (end 179.655 99.1621) (width 0.2) (layer "F.Cu") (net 2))
 (segment (start 127.1588 87.9475) (end 128.1871 88.9758) (width 0.2) (layer "F.Cu") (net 2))
 (segment (start 178.1675 98.0921) (end 179.2375 99.1621) (width 0.2) (layer "F.Cu") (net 2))
 (segment (start 128.1871 88.9758) (end 128.1871 91.3876) (width 0.2) (layer "F.Cu") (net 2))
 (segment (start 149.9064 95.3509) (end 146.38 91.8245) (width 0.2) (layer "F.Cu") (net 10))
 (segment (start 177.9663 95.3509) (end 149.9064 95.3509) (width 0.2) (layer "F.Cu") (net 10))
 (segment (start 146.38 88.1187) (end 146.2088 87.9475) (width 0.2) (layer "F.Cu") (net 10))
 (segment (start 146.38 91.8245) (end 146.38 88.1187) (width 0.2) (layer "F.Cu") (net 10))
 (segment (start 179.2375 96.6221) (end 177.9663 95.3509) (width 0.2) (layer "F.Cu") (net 10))
 (segment (start 179.2375 96.6221) (end 180.0725 96.6221) (width 0.2) (layer "F.Cu") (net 10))
 (segment (start 181.6372 99.9148) (end 179.2846 102.2674) (width 0.2) (layer "F.Cu") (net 11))
 (segment (start 179.2375 94.0821) (end 180.0725 94.0821) (width 0.2) (layer "F.Cu") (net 11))
 (segment (start 179.2846 102.2674) (end 131.8889 102.2674) (width 0.2) (layer "F.Cu") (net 11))
 (segment (start 131.8889 102.2674) (end 127.1588 106.9975) (width 0.2) (layer "F.Cu") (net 11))
 (segment (start 181.6372 95.6468) (end 181.6372 99.9148) (width 0.2) (layer "F.Cu") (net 11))
 (segment (start 180.0725 94.0821) (end 181.6372 95.6468) (width 0.2) (layer "F.Cu") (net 11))
 (segment (start 180.0725 91.5421) (end 179.2375 91.5421) (width 0.2) (layer "F.Cu") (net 12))
 (segment (start 151.755 92.6705) (end 150.4307 93.9948) (width 0.2) (layer "F.Cu") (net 12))
 (segment (start 149.4431 93.9932) (end 149.4431 93.9948) (width 0.2) (layer "F.Cu") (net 12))
 (segment (start 178.1091 92.6705) (end 151.755 92.6705) (width 0.2) (layer "F.Cu") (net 12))
 (segment (start 150.4307 93.9948) (end 149.4431 93.9948) (width 0.2) (layer "F.Cu") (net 12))
 (segment (start 179.2375 91.5421) (end 178.1091 92.6705) (width 0.2) (layer "F.Cu") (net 12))
 (segment (start 149.4431 93.9948) (end 149.4431 93.9932) (width 0.2) (layer "F.Cu") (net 12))
 (via (at 149.4431 93.9948) (size 0.6) (drill 0.3) (layers "F.Cu" "B.Cu") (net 12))
 (segment (start 149.4431 93.9948) (end 146.2088 97.2291) (width 0.2) (layer "B.Cu") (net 12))
 (segment (start 149.4431 93.9932) (end 149.4431 93.9948) (width 0.2) (layer "B.Cu") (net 12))
 (segment (start 146.2088 97.2291) (end 146.2088 106.9975) (width 0.2) (layer "B.Cu") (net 12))
 (segment (start 149.4431 93.9948) (end 149.4431 93.9932) (width 0.2) (layer "B.Cu") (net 12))
 (segment (start 163.9975 89.0021) (end 163.1625 89.0021) (width 0.2) (layer "F.Cu") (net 5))
 (segment (start 163.9975 86.4621) (end 163.1625 86.4621) (width 0.2) (layer "F.Cu") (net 4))
 (segment (start 163.1625 83.9221) (end 163.9975 83.9221) (width 0.2) (layer "F.Cu") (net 3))
 (segment (start 163.9975 99.1621) (end 163.1625 99.1621) (width 0.2) (layer "F.Cu") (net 9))
 (segment (start 163.1625 96.6221) (end 163.9975 96.6221) (width 0.2) (layer "F.Cu") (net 8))
 (segment (start 163.9975 91.5421) (end 163.1625 91.5421) (width 0.2) (layer "F.Cu") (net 6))
 (segment (start 180.0725 89.0021) (end 179.2375 89.0021) (width 0.2) (layer "F.Cu") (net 13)))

